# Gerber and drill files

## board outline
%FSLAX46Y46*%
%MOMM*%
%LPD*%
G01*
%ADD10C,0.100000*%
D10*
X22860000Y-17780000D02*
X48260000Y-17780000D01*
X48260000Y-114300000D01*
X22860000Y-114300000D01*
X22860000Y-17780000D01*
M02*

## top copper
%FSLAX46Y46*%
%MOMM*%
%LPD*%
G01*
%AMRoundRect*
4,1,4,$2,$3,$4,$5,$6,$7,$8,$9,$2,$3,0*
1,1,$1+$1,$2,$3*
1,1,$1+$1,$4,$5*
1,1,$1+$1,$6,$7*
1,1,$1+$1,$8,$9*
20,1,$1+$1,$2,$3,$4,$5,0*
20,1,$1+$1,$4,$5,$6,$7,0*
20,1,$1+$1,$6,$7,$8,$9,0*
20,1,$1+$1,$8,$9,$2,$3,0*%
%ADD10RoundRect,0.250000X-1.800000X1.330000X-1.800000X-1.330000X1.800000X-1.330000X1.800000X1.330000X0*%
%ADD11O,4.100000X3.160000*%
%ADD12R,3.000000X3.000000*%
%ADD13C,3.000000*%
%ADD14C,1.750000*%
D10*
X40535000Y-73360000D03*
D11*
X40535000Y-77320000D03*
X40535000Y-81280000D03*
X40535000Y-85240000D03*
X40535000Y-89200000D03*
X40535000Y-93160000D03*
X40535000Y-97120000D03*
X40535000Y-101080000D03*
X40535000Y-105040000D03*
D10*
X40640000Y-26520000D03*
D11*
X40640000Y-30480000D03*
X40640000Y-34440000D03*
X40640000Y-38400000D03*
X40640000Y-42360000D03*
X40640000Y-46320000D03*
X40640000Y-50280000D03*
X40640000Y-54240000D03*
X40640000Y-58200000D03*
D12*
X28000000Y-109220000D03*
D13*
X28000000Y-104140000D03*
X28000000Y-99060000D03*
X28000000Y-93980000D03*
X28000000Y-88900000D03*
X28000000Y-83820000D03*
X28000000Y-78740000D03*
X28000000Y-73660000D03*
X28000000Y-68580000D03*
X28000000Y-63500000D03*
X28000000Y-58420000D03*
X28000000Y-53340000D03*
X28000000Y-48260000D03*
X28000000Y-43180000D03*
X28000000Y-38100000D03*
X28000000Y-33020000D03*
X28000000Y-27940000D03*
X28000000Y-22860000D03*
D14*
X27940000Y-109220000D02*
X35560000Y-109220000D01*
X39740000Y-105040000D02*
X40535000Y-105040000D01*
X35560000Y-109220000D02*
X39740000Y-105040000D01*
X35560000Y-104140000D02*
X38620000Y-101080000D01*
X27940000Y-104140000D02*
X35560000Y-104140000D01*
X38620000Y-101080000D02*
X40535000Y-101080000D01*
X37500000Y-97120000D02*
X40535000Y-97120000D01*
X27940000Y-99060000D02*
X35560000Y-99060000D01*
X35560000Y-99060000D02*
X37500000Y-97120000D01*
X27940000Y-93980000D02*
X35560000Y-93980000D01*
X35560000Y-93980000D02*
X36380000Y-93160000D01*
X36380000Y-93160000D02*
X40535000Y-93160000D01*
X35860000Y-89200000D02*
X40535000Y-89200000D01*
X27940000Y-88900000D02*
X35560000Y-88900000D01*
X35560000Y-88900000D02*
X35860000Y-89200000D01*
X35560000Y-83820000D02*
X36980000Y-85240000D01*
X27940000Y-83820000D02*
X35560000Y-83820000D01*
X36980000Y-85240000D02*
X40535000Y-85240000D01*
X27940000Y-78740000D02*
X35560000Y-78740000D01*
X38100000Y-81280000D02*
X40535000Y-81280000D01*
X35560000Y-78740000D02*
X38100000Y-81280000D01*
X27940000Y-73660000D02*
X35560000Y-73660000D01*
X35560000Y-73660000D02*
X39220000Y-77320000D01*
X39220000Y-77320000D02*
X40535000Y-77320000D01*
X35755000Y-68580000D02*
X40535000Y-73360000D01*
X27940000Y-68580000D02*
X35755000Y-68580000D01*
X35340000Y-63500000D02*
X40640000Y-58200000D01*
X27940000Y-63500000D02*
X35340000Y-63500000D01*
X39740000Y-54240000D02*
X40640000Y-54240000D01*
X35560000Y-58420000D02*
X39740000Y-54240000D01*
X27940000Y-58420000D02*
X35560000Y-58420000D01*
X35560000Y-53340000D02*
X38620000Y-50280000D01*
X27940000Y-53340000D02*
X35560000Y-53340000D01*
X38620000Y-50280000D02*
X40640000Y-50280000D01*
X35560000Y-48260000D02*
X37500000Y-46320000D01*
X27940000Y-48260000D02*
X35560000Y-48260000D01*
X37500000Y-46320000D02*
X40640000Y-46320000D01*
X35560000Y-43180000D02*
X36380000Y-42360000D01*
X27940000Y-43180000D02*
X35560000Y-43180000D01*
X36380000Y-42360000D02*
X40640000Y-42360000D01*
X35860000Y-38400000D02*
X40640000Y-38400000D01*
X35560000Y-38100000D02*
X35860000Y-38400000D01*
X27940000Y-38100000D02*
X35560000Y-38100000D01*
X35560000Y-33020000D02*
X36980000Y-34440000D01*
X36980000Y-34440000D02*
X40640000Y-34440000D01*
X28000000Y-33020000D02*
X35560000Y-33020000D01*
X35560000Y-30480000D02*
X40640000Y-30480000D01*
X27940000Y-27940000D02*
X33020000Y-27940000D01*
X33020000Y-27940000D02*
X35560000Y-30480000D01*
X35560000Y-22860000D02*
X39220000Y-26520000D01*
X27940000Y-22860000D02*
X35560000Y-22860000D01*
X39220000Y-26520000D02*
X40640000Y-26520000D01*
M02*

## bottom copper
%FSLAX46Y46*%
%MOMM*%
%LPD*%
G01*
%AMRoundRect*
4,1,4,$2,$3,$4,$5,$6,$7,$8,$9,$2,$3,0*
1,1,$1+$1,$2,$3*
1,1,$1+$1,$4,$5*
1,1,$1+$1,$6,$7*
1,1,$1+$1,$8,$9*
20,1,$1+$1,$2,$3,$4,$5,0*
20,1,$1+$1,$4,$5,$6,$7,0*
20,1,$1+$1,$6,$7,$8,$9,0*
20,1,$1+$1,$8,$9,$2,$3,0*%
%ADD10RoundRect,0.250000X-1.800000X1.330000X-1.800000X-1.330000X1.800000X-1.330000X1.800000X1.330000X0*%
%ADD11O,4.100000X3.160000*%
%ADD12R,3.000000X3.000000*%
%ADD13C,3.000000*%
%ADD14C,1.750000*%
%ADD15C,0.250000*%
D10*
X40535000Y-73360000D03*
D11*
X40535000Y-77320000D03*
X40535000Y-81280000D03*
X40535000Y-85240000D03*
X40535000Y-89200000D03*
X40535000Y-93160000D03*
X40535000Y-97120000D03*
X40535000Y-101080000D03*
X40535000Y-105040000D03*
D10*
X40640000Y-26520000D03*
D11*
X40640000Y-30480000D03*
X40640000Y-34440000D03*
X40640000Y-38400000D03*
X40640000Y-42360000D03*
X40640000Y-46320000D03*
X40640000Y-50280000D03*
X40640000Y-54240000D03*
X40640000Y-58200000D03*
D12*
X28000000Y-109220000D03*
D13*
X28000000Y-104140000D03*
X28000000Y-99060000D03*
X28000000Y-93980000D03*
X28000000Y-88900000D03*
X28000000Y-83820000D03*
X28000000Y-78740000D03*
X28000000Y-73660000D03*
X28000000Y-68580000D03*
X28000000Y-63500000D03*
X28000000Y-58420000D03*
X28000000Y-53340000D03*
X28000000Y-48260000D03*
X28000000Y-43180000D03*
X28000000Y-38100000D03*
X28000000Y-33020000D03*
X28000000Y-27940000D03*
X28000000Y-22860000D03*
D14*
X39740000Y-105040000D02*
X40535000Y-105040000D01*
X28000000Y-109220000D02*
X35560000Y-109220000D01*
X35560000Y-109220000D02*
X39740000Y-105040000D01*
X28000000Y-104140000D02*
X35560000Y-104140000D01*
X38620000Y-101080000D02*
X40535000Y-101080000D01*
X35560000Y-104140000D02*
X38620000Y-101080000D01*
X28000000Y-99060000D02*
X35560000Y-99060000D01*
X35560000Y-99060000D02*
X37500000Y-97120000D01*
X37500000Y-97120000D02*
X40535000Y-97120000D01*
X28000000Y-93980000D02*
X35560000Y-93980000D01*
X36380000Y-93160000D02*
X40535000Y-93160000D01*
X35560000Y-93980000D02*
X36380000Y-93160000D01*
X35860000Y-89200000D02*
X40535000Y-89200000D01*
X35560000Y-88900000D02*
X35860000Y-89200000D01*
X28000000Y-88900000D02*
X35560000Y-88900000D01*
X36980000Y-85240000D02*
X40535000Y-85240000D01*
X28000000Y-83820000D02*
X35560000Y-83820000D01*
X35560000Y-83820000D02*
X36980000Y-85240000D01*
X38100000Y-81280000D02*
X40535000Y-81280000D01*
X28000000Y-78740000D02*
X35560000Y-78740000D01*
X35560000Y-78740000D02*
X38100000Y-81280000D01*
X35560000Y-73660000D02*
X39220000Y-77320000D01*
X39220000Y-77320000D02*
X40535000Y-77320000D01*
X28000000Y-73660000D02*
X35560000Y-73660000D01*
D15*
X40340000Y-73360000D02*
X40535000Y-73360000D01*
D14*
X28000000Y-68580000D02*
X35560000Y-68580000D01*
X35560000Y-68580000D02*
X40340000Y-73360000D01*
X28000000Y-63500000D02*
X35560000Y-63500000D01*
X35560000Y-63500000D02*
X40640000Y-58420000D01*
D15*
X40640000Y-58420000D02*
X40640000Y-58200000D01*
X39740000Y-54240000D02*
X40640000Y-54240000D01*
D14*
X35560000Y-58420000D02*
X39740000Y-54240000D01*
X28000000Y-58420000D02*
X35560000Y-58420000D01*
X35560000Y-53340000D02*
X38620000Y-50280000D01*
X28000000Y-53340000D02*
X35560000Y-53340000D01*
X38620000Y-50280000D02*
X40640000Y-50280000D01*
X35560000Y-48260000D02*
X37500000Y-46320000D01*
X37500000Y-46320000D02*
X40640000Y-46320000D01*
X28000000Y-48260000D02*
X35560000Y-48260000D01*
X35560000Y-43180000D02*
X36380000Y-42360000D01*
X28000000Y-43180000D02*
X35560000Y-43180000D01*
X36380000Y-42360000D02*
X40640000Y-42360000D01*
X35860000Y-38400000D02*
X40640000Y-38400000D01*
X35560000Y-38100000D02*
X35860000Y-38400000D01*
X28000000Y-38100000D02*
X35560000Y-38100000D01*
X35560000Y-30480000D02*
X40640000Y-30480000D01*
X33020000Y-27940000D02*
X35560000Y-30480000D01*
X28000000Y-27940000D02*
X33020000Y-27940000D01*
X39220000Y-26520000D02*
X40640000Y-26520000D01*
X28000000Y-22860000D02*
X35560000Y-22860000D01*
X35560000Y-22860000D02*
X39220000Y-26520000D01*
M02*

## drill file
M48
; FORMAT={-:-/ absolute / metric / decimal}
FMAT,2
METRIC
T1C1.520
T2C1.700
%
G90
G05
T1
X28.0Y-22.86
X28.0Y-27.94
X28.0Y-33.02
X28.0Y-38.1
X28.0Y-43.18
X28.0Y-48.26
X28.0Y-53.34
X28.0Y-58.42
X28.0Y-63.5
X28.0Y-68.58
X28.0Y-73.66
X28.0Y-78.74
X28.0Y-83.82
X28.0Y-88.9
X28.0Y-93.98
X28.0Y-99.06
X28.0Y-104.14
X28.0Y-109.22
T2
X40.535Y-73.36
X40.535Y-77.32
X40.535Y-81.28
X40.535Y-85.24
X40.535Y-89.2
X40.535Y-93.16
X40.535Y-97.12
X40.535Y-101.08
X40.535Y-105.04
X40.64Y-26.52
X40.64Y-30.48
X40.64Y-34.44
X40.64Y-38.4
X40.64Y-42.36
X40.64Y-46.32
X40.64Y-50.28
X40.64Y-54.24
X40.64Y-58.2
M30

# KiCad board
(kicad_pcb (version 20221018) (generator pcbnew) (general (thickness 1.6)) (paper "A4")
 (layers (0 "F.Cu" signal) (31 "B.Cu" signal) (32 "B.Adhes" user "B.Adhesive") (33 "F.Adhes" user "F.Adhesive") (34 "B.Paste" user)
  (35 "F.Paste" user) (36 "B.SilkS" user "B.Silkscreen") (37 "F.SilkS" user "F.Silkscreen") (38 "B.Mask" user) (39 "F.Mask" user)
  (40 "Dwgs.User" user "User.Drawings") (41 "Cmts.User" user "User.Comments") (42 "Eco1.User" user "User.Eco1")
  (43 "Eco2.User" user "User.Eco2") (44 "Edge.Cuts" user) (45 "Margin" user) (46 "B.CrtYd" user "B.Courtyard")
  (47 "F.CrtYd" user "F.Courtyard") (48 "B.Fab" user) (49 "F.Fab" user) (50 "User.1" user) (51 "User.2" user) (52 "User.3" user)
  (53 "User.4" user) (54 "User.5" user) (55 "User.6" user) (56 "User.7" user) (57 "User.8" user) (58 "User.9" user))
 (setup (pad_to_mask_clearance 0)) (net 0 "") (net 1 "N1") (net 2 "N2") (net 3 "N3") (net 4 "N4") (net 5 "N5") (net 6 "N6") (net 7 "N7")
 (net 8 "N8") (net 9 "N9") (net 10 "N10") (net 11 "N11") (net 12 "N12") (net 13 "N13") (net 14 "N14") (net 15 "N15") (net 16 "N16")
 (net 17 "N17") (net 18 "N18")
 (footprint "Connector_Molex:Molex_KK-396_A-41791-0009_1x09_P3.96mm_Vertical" (layer "F.Cu") (at 40.535 73.36 -90)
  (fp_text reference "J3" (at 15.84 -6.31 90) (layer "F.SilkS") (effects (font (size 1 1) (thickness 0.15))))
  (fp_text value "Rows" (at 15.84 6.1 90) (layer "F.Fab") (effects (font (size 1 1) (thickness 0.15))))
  (pad "1" thru_hole roundrect (at 0 0 270) (size 3.16 4.1) (drill 1.7) (layers "*.Cu" "*.Mask") (roundrect_rratio 0.07911392405)
   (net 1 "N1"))
  (pad "2" thru_hole oval (at 3.96 0 270) (size 3.16 4.1) (drill 1.7) (layers "*.Cu" "*.Mask") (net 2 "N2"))
  (pad "3" thru_hole oval (at 7.92 0 270) (size 3.16 4.1) (drill 1.7) (layers "*.Cu" "*.Mask") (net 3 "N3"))
  (pad "4" thru_hole oval (at 11.88 0 270) (size 3.16 4.1) (drill 1.7) (layers "*.Cu" "*.Mask") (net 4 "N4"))
  (pad "5" thru_hole oval (at 15.84 0 270) (size 3.16 4.1) (drill 1.7) (layers "*.Cu" "*.Mask") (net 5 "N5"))
  (pad "6" thru_hole oval (at 19.8 0 270) (size 3.16 4.1) (drill 1.7) (layers "*.Cu" "*.Mask") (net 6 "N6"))
  (pad "7" thru_hole oval (at 23.76 0 270) (size 3.16 4.1) (drill 1.7) (layers "*.Cu" "*.Mask") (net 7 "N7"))
  (pad "8" thru_hole oval (at 27.72 0 270) (size 3.16 4.1) (drill 1.7) (layers "*.Cu" "*.Mask") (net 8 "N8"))
  (pad "9" thru_hole oval (at 31.68 0 270) (size 3.16 4.1) (drill 1.7) (layers "*.Cu" "*.Mask") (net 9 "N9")))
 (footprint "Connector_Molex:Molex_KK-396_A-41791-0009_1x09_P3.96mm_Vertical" (layer "F.Cu") (at 40.64 26.52 -90)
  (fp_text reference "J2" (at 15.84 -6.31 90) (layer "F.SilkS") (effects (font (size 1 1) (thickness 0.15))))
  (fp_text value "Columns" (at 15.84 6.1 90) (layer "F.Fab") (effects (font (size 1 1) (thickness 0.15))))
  (pad "1" thru_hole roundrect (at 0 0 270) (size 3.16 4.1) (drill 1.7) (layers "*.Cu" "*.Mask") (roundrect_rratio 0.07911392405)
   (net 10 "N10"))
  (pad "2" thru_hole oval (at 3.96 0 270) (size 3.16 4.1) (drill 1.7) (layers "*.Cu" "*.Mask") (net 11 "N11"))
  (pad "3" thru_hole oval (at 7.92 0 270) (size 3.16 4.1) (drill 1.7) (layers "*.Cu" "*.Mask") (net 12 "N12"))
  (pad "4" thru_hole oval (at 11.88 0 270) (size 3.16 4.1) (drill 1.7) (layers "*.Cu" "*.Mask") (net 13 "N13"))
  (pad "5" thru_hole oval (at 15.84 0 270) (size 3.16 4.1) (drill 1.7) (layers "*.Cu" "*.Mask") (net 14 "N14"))
  (pad "6" thru_hole oval (at 19.8 0 270) (size 3.16 4.1) (drill 1.7) (layers "*.Cu" "*.Mask") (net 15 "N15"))
  (pad "7" thru_hole oval (at 23.76 0 270) (size 3.16 4.1) (drill 1.7) (layers "*.Cu" "*.Mask") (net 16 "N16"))
  (pad "8" thru_hole oval (at 27.72 0 270) (size 3.16 4.1) (drill 1.7) (layers "*.Cu" "*.Mask") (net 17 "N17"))
  (pad "9" thru_hole oval (at 31.68 0 270) (size 3.16 4.1) (drill 1.7) (layers "*.Cu" "*.Mask") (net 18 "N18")))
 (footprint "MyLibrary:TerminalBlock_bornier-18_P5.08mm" (layer "F.Cu") (at 28 109.22 90)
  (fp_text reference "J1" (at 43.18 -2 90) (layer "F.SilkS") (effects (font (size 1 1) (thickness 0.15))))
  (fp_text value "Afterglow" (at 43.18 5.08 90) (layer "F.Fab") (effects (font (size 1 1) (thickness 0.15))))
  (pad "1" thru_hole rect (at 0 0 90) (size 3 3) (drill 1.52) (layers "*.Cu" "*.Mask") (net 9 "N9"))
  (pad "2" thru_hole circle (at 5.08 0 90) (size 3 3) (drill 1.52) (layers "*.Cu" "*.Mask") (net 8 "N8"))
  (pad "3" thru_hole circle (at 10.16 0 90) (size 3 3) (drill 1.52) (layers "*.Cu" "*.Mask") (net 7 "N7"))
  (pad "4" thru_hole circle (at 15.24 0 90) (size 3 3) (drill 1.52) (layers "*.Cu" "*.Mask") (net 6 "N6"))
  (pad "5" thru_hole circle (at 20.32 0 90) (size 3 3) (drill 1.52) (layers "*.Cu" "*.Mask") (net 5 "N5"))
  (pad "6" thru_hole circle (at 25.4 0 90) (size 3 3) (drill 1.52) (layers "*.Cu" "*.Mask") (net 4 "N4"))
  (pad "7" thru_hole circle (at 30.48 0 90) (size 3 3) (drill 1.52) (layers "*.Cu" "*.Mask") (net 3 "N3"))
  (pad "8" thru_hole circle (at 35.56 0 90) (size 3 3) (drill 1.52) (layers "*.Cu" "*.Mask") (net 2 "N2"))
  (pad "9" thru_hole circle (at 40.64 0 90) (size 3 3) (drill 1.52) (layers "*.Cu" "*.Mask") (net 1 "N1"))
  (pad "10" thru_hole circle (at 45.72 0 90) (size 3 3) (drill 1.52) (layers "*.Cu" "*.Mask") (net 18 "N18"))
  (pad "11" thru_hole circle (at 50.8 0 90) (size 3 3) (drill 1.52) (layers "*.Cu" "*.Mask") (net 17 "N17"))
  (pad "12" thru_hole circle (at 55.88 0 90) (size 3 3) (drill 1.52) (layers "*.Cu" "*.Mask") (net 16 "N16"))
  (pad "13" thru_hole circle (at 60.96 0 90) (size 3 3) (drill 1.52) (layers "*.Cu" "*.Mask") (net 15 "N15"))
  (pad "14" thru_hole circle (at 66.04 0 90) (size 3 3) (drill 1.52) (layers "*.Cu" "*.Mask") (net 14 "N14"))
  (pad "15" thru_hole circle (at 71.12 0 90) (size 3 3) (drill 1.52) (layers "*.Cu" "*.Mask") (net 13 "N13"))
  (pad "16" thru_hole circle (at 76.2 0 90) (size 3 3) (drill 1.52) (layers "*.Cu" "*.Mask") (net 12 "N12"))
  (pad "17" thru_hole circle (at 81.28 0 90) (size 3 3) (drill 1.52) (layers "*.Cu" "*.Mask") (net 11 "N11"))
  (pad "18" thru_hole circle (at 86.36 0 90) (size 3 3) (drill 1.52) (layers "*.Cu" "*.Mask") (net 10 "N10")))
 (gr_rect (start 22.86 17.78) (end 48.26 114.3) (stroke (width 0.1) (type default)) (fill none) (layer "Edge.Cuts"))
 (segment (start 27.94 109.22) (end 35.56 109.22) (width 1.75) (layer "F.Cu") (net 9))
 (segment (start 39.74 105.04) (end 40.535 105.04) (width 1.75) (layer "F.Cu") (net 9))
 (segment (start 35.56 109.22) (end 39.74 105.04) (width 1.75) (layer "F.Cu") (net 9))
 (segment (start 39.74 105.04) (end 40.535 105.04) (width 1.75) (layer "B.Cu") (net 9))
 (segment (start 28 109.22) (end 35.56 109.22) (width 1.75) (layer "B.Cu") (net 9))
 (segment (start 35.56 109.22) (end 39.74 105.04) (width 1.75) (layer "B.Cu") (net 9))
 (segment (start 35.56 104.14) (end 38.62 101.08) (width 1.75) (layer "F.Cu") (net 8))
 (segment (start 27.94 104.14) (end 35.56 104.14) (width 1.75) (layer "F.Cu") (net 8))
 (segment (start 38.62 101.08) (end 40.535 101.08) (width 1.75) (layer "F.Cu") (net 8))
 (segment (start 28 104.14) (end 35.56 104.14) (width 1.75) (layer "B.Cu") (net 8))
 (segment (start 38.62 101.08) (end 40.535 101.08) (width 1.75) (layer "B.Cu") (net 8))
 (segment (start 35.56 104.14) (end 38.62 101.08) (width 1.75) (layer "B.Cu") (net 8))
 (segment (start 37.5 97.12) (end 40.535 97.12) (width 1.75) (layer "F.Cu") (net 7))
 (segment (start 27.94 99.06) (end 35.56 99.06) (width 1.75) (layer "F.Cu") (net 7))
 (segment (start 35.56 99.06) (end 37.5 97.12) (width 1.75) (layer "F.Cu") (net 7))
 (segment (start 28 99.06) (end 35.56 99.06) (width 1.75) (layer "B.Cu") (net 7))
 (segment (start 35.56 99.06) (end 37.5 97.12) (width 1.75) (layer "B.Cu") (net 7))
 (segment (start 37.5 97.12) (end 40.535 97.12) (width 1.75) (layer "B.Cu") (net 7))
 (segment (start 27.94 93.98) (end 35.56 93.98) (width 1.75) (layer "F.Cu") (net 6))
 (segment (start 35.56 93.98) (end 36.38 93.16) (width 1.75) (layer "F.Cu") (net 6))
 (segment (start 36.38 93.16) (end 40.535 93.16) (width 1.75) (layer "F.Cu") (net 6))
 (segment (start 28 93.98) (end 35.56 93.98) (width 1.75) (layer "B.Cu") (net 6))
 (segment (start 36.38 93.16) (end 40.535 93.16) (width 1.75) (layer "B.Cu") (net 6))
 (segment (start 35.56 93.98) (end 36.38 93.16) (width 1.75) (layer "B.Cu") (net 6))
 (segment (start 35.86 89.2) (end 40.535 89.2) (width 1.75) (layer "F.Cu") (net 5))
 (segment (start 27.94 88.9) (end 35.56 88.9) (width 1.75) (layer "F.Cu") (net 5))
 (segment (start 35.56 88.9) (end 35.86 89.2) (width 1.75) (layer "F.Cu") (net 5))
 (segment (start 35.86 89.2) (end 40.535 89.2) (width 1.75) (layer "B.Cu") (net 5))
 (segment (start 35.56 88.9) (end 35.86 89.2) (width 1.75) (layer "B.Cu") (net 5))
 (segment (start 28 88.9) (end 35.56 88.9) (width 1.75) (layer "B.Cu") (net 5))
 (segment (start 35.56 83.82) (end 36.98 85.24) (width 1.75) (layer "F.Cu") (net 4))
 (segment (start 27.94 83.82) (end 35.56 83.82) (width 1.75) (layer "F.Cu") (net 4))
 (segment (start 36.98 85.24) (end 40.535 85.24) (width 1.75) (layer "F.Cu") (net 4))
 (segment (start 36.98 85.24) (end 40.535 85.24) (width 1.75) (layer "B.Cu") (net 4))
 (segment (start 28 83.82) (end 35.56 83.82) (width 1.75) (layer "B.Cu") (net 4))
 (segment (start 35.56 83.82) (end 36.98 85.24) (width 1.75) (layer "B.Cu") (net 4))
 (segment (start 27.94 78.74) (end 35.56 78.74) (width 1.75) (layer "F.Cu") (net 3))
 (segment (start 38.1 81.28) (end 40.535 81.28) (width 1.75) (layer "F.Cu") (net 3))
 (segment (start 35.56 78.74) (end 38.1 81.28) (width 1.75) (layer "F.Cu") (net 3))
 (segment (start 38.1 81.28) (end 40.535 81.28) (width 1.75) (layer "B.Cu") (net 3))
 (segment (start 28 78.74) (end 35.56 78.74) (width 1.75) (layer "B.Cu") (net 3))
 (segment (start 35.56 78.74) (end 38.1 81.28) (width 1.75) (layer "B.Cu") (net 3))
 (segment (start 27.94 73.66) (end 35.56 73.66) (width 1.75) (layer "F.Cu") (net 2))
 (segment (start 35.56 73.66) (end 39.22 77.32) (width 1.75) (layer "F.Cu") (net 2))
 (segment (start 39.22 77.32) (end 40.535 77.32) (width 1.75) (layer "F.Cu") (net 2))
 (segment (start 35.56 73.66) (end 39.22 77.32) (width 1.75) (layer "B.Cu") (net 2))
 (segment (start 39.22 77.32) (end 40.535 77.32) (width 1.75) (layer "B.Cu") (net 2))
 (segment (start 28 73.66) (end 35.56 73.66) (width 1.75) (layer "B.Cu") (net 2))
 (segment (start 35.755 68.58) (end 40.535 73.36) (width 1.75) (layer "F.Cu") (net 1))
 (segment (start 27.94 68.58) (end 35.755 68.58) (width 1.75) (layer "F.Cu") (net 1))
 (segment (start 40.34 73.36) (end 40.535 73.36) (width 0.25) (layer "B.Cu") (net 1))
 (segment (start 28 68.58) (end 35.56 68.58) (width 1.75) (layer "B.Cu") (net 1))
 (segment (start 35.56 68.58) (end 40.34 73.36) (width 1.75) (layer "B.Cu") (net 1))
 (segment (start 35.34 63.5) (end 40.64 58.2) (width 1.75) (layer "F.Cu") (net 18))
 (segment (start 27.94 63.5) (end 35.34 63.5) (width 1.75) (layer "F.Cu") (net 18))
 (segment (start 28 63.5) (end 35.56 63.5) (width 1.75) (layer "B.Cu") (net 18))
 (segment (start 35.56 63.5) (end 40.64 58.42) (width 1.75) (layer "B.Cu") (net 18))
 (segment (start 40.64 58.42) (end 40.64 58.2) (width 0.25) (layer "B.Cu") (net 18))
 (segment (start 39.74 54.24) (end 40.64 54.24) (width 1.75) (layer "F.Cu") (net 17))
 (segment (start 35.56 58.42) (end 39.74 54.24) (width 1.75) (layer "F.Cu") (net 17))
 (segment (start 27.94 58.42) (end 35.56 58.42) (width 1.75) (layer "F.Cu") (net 17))
 (segment (start 39.74 54.24) (end 40.64 54.24) (width 0.25) (layer "B.Cu") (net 17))
 (segment (start 35.56 58.42) (end 39.74 54.24) (width 1.75) (layer "B.Cu") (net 17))
 (segment (start 28 58.42) (end 35.56 58.42) (width 1.75) (layer "B.Cu") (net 17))
 (segment (start 35.56 53.34) (end 38.62 50.28) (width 1.75) (layer "F.Cu") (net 16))
 (segment (start 27.94 53.34) (end 35.56 53.34) (width 1.75) (layer "F.Cu") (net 16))
 (segment (start 38.62 50.28) (end 40.64 50.28) (width 1.75) (layer "F.Cu") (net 16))
 (segment (start 35.56 53.34) (end 38.62 50.28) (width 1.75) (layer "B.Cu") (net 16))
 (segment (start 28 53.34) (end 35.56 53.34) (width 1.75) (layer "B.Cu") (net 16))
 (segment (start 38.62 50.28) (end 40.64 50.28) (width 1.75) (layer "B.Cu") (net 16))
 (segment (start 35.56 48.26) (end 37.5 46.32) (width 1.75) (layer "F.Cu") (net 15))
 (segment (start 27.94 48.26) (end 35.56 48.26) (width 1.75) (layer "F.Cu") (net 15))
 (segment (start 37.5 46.32) (end 40.64 46.32) (width 1.75) (layer "F.Cu") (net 15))
 (segment (start 35.56 48.26) (end 37.5 46.32) (width 1.75) (layer "B.Cu") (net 15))
 (segment (start 37.5 46.32) (end 40.64 46.32) (width 1.75) (layer "B.Cu") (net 15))
 (segment (start 28 48.26) (end 35.56 48.26) (width 1.75) (layer "B.Cu") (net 15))
 (segment (start 35.56 43.18) (end 36.38 42.36) (width 1.75) (layer "F.Cu") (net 14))
 (segment (start 27.94 43.18) (end 35.56 43.18) (width 1.75) (layer "F.Cu") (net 14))
 (segment (start 36.38 42.36) (end 40.64 42.36) (width 1.75) (layer "F.Cu") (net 14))
 (segment (start 35.56 43.18) (end 36.38 42.36) (width 1.75) (layer "B.Cu") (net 14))
 (segment (start 28 43.18) (end 35.56 43.18) (width 1.75) (layer "B.Cu") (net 14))
 (segment (start 36.38 42.36) (end 40.64 42.36) (width 1.75) (layer "B.Cu") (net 14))
 (segment (start 35.86 38.4) (end 40.64 38.4) (width 1.75) (layer "F.Cu") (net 13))
 (segment (start 35.56 38.1) (end 35.86 38.4) (width 1.75) (layer "F.Cu") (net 13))
 (segment (start 27.94 38.1) (end 35.56 38.1) (width 1.75) (layer "F.Cu") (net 13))
 (segment (start 35.86 38.4) (end 40.64 38.4) (width 1.75) (layer "B.Cu") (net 13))
 (segment (start 35.56 38.1) (end 35.86 38.4) (width 1.75) (layer "B.Cu") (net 13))
 (segment (start 28 38.1) (end 35.56 38.1) (width 1.75) (layer "B.Cu") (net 13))
 (segment (start 35.56 33.02) (end 36.98 34.44) (width 1.75) (layer "F.Cu") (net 12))
 (segment (start 36.98 34.44) (end 40.64 34.44) (width 1.75) (layer "F.Cu") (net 12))
 (segment (start 28 33.02) (end 35.56 33.02) (width 1.75) (layer "F.Cu") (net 12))
 (segment (start 35.56 30.48) (end 40.64 30.48) (width 1.75) (layer "F.Cu") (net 11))
 (segment (start 27.94 27.94) (end 33.02 27.94) (width 1.75) (layer "F.Cu") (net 11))
 (segment (start 33.02 27.94) (end 35.56 30.48) (width 1.75) (layer "F.Cu") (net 11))
 (segment (start 35.56 30.48) (end 40.64 30.48) (width 1.75) (layer "B.Cu") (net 11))
 (segment (start 33.02 27.94) (end 35.56 30.48) (width 1.75) (layer "B.Cu") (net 11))
 (segment (start 28 27.94) (end 33.02 27.94) (width 1.75) (layer "B.Cu") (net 11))
 (segment (start 35.56 22.86) (end 39.22 26.52) (width 1.75) (layer "F.Cu") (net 10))
 (segment (start 27.94 22.86) (end 35.56 22.86) (width 1.75) (layer "F.Cu") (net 10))
 (segment (start 39.22 26.52) (end 40.64 26.52) (width 1.75) (layer "F.Cu") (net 10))
 (segment (start 39.22 26.52) (end 40.64 26.52) (width 1.75) (layer "B.Cu") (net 10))
 (segment (start 28 22.86) (end 35.56 22.86) (width 1.75) (layer "B.Cu") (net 10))
 (segment (start 35.56 22.86) (end 39.22 26.52) (width 1.75) (layer "B.Cu") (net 10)))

